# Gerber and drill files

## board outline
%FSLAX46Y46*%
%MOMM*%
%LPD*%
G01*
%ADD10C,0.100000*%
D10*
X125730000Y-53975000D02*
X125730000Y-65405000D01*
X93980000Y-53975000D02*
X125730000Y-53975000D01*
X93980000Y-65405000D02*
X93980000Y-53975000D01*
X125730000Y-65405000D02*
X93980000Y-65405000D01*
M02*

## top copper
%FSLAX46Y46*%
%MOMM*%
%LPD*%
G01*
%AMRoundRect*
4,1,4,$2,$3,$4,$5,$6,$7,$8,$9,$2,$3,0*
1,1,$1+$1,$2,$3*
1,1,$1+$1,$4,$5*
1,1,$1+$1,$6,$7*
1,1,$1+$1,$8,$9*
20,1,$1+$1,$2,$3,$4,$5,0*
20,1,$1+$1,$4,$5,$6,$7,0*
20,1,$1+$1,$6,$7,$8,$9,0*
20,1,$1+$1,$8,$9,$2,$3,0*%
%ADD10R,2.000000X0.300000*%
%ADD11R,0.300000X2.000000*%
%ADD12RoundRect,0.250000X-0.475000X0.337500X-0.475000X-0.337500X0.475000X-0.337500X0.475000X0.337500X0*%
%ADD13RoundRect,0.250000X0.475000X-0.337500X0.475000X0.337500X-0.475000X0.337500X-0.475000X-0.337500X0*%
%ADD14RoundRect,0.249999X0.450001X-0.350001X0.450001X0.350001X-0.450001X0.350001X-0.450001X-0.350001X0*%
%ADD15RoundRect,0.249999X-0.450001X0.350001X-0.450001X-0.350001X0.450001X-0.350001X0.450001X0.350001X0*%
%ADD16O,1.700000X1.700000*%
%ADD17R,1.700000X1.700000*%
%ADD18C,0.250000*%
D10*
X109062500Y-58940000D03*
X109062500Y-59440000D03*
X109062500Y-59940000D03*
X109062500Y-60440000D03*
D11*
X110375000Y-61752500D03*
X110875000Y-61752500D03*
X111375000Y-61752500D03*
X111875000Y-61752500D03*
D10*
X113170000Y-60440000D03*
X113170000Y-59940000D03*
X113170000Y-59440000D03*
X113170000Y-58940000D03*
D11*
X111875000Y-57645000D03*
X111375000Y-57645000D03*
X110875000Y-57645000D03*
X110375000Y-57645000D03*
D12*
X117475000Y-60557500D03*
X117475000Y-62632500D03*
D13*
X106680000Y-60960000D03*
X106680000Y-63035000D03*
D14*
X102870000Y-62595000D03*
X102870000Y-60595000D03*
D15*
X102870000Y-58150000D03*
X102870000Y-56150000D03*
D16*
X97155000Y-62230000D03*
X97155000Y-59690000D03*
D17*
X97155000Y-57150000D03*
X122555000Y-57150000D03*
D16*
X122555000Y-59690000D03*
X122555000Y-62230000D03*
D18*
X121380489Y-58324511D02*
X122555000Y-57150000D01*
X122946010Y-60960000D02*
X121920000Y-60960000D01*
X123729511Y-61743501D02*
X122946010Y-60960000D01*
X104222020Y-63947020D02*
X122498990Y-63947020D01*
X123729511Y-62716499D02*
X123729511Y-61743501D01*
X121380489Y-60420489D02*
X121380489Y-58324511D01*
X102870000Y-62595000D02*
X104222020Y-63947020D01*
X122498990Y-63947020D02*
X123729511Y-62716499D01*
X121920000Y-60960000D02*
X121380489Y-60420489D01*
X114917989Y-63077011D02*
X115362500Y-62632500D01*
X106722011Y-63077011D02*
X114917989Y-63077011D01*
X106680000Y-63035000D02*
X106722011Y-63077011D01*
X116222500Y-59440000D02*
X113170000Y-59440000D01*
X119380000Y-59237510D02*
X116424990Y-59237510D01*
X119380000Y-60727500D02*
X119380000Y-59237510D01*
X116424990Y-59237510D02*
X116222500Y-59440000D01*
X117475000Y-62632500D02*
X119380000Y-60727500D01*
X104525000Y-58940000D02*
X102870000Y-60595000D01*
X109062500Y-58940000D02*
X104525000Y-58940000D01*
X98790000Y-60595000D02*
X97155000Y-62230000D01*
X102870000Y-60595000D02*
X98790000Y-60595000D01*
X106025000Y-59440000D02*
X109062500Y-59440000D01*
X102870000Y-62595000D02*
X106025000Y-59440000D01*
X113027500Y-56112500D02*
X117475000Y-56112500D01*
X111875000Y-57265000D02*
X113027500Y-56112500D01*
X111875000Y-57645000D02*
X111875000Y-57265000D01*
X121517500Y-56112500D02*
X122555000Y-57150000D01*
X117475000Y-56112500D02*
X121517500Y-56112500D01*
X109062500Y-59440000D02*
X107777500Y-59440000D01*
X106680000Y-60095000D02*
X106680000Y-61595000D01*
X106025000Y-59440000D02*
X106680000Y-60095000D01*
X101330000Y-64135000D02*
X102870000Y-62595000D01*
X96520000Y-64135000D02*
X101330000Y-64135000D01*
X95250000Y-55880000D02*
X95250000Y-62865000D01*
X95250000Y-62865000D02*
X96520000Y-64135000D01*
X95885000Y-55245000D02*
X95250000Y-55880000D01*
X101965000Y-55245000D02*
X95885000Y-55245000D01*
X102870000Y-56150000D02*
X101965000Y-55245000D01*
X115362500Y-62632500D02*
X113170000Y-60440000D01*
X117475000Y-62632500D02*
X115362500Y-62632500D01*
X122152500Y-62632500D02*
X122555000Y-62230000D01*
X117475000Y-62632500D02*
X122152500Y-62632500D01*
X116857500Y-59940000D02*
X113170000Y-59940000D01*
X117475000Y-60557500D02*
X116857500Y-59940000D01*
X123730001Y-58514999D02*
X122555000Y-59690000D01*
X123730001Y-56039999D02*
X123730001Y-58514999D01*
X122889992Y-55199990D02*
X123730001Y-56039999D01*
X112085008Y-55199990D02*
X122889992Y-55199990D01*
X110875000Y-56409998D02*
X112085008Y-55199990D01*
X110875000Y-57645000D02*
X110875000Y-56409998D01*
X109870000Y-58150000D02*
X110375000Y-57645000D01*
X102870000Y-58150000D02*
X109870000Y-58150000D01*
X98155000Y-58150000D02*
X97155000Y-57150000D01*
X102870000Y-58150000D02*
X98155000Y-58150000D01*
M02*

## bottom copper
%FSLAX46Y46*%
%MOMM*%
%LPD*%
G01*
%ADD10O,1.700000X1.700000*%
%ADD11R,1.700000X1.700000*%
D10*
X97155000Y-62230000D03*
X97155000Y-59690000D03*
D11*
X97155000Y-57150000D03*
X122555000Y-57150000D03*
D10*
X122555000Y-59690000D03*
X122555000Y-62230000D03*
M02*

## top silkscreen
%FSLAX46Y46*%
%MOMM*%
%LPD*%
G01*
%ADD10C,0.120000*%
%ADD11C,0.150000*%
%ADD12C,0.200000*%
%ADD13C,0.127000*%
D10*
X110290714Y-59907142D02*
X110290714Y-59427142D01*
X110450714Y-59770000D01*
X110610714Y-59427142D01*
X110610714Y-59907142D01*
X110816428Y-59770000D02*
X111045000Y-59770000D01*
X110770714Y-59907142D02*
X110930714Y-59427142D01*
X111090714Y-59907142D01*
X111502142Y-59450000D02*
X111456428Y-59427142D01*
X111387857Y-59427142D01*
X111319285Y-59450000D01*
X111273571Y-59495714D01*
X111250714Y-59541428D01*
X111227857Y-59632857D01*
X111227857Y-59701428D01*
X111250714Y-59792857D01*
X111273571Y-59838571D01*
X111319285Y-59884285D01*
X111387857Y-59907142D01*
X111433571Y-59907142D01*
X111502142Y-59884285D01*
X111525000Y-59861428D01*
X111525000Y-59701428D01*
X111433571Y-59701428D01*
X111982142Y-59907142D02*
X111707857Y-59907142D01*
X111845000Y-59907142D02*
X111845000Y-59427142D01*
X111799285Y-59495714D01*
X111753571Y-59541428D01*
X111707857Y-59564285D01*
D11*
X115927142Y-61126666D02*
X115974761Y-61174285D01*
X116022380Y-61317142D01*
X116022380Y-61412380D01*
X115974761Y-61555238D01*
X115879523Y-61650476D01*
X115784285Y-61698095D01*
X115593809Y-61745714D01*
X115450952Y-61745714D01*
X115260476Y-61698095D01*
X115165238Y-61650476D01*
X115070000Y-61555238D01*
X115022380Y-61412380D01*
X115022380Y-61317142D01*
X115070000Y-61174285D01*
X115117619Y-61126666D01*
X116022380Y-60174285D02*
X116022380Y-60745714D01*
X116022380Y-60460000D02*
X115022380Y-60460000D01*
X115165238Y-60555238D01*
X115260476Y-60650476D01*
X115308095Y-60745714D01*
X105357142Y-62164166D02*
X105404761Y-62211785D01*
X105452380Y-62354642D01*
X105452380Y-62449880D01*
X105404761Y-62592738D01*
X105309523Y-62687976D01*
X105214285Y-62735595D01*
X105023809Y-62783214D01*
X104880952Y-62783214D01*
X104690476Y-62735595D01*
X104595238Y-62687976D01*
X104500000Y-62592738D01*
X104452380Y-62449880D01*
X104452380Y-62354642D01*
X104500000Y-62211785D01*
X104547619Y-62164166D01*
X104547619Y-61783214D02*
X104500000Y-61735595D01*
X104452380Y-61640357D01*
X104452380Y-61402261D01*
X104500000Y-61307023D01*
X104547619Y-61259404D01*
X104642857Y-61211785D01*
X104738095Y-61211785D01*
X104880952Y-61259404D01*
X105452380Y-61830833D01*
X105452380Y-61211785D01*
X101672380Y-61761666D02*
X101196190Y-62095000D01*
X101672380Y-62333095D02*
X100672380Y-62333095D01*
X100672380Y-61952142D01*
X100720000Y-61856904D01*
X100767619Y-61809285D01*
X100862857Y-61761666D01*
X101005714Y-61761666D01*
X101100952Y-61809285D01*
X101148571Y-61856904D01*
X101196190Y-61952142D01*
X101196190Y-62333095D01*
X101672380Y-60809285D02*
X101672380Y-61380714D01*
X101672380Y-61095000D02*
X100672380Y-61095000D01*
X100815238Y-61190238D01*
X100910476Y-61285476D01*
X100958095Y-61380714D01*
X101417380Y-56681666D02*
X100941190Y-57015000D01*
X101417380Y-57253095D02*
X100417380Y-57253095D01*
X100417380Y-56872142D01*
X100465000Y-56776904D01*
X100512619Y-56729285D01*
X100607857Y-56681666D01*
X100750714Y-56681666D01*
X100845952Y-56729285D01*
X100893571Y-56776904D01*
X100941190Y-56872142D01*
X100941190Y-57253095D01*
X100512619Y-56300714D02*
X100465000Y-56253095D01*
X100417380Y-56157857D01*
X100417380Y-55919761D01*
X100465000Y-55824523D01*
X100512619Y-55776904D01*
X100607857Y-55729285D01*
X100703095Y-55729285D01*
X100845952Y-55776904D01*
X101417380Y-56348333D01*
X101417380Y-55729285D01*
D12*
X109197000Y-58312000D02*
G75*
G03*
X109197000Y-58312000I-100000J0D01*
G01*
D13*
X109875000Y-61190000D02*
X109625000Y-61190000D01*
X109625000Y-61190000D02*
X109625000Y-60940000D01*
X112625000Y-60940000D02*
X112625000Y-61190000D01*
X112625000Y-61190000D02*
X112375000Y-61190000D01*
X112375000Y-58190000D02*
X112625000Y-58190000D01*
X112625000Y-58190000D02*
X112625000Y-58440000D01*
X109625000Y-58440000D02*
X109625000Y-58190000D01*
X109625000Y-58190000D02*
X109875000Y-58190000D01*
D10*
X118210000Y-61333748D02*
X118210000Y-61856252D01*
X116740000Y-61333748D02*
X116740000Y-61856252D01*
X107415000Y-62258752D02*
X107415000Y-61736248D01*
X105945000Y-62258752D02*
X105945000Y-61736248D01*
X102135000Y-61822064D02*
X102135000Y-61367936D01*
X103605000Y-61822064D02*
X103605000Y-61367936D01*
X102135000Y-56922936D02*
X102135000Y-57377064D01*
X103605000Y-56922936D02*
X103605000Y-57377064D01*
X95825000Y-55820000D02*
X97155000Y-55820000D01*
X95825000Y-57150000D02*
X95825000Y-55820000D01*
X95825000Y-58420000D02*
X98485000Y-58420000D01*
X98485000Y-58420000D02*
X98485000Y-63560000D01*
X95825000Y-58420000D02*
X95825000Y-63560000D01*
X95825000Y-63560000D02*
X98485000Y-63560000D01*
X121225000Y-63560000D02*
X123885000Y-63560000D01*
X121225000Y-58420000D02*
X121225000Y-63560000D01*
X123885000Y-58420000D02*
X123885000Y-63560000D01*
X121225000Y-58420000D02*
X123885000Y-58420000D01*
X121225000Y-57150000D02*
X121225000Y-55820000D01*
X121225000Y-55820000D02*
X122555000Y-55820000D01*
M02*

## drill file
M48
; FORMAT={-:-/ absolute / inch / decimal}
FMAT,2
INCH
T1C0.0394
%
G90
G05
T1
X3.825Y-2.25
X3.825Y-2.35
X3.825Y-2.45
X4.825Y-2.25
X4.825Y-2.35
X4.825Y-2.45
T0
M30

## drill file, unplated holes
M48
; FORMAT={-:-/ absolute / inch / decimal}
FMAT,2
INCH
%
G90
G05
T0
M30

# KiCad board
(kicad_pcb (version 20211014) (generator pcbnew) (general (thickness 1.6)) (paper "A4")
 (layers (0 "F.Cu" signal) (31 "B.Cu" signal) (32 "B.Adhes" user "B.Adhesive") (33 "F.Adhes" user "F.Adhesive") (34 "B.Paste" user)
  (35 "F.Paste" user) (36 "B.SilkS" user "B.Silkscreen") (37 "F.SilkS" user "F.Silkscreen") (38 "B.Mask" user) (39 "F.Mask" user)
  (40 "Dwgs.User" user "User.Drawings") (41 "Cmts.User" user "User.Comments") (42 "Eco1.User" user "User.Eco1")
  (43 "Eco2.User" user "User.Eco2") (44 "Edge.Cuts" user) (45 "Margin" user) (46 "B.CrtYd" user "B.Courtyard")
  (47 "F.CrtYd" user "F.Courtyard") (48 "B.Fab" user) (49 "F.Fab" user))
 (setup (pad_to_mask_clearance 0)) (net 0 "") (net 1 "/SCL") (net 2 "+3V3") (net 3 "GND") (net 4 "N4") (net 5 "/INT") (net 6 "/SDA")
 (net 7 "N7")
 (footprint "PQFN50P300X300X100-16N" (layer "F.Cu") (at 111.125 59.69)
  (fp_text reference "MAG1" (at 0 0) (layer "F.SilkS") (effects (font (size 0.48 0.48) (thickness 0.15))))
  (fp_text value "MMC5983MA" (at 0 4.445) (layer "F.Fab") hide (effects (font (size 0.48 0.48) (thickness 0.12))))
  (fp_line (start 1.5 1.5) (end 1.25 1.5) (layer "F.SilkS") (width 0.127))
  (fp_line (start 1.5 -1.5) (end 1.5 -1.25) (layer "F.SilkS") (width 0.127))
  (fp_line (start 1.25 -1.5) (end 1.5 -1.5) (layer "F.SilkS") (width 0.127))
  (fp_line (start -1.5 -1.5) (end -1.25 -1.5) (layer "F.SilkS") (width 0.127))
  (fp_line (start -1.5 -1.25) (end -1.5 -1.5) (layer "F.SilkS") (width 0.127))
  (fp_line (start 1.5 1.25) (end 1.5 1.5) (layer "F.SilkS") (width 0.127))
  (fp_line (start -1.25 1.5) (end -1.5 1.5) (layer "F.SilkS") (width 0.127))
  (fp_line (start -1.5 1.5) (end -1.5 1.25) (layer "F.SilkS") (width 0.127))
  (fp_circle (center -2.028 -1.378) (end -1.928 -1.378) (layer "F.SilkS") (width 0.2) (fill none))
  (pad "1" smd rect locked (at -2.0625 -0.75) (size 2 0.3) (layers "F.Cu" "F.Paste" "F.Mask") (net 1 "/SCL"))
  (pad "2" smd rect locked (at -2.0625 -0.25) (size 2 0.3) (layers "F.Cu" "F.Paste" "F.Mask") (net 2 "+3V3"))
  (pad "3" smd rect locked (at -2.0625 0.25) (size 2 0.3) (layers "F.Cu" "F.Paste" "F.Mask"))
  (pad "4" smd rect locked (at -2.0625 0.75) (size 2 0.3) (layers "F.Cu" "F.Paste" "F.Mask"))
  (pad "5" smd rect locked (at -0.75 2.0625) (size 0.3 2) (layers "F.Cu" "F.Paste" "F.Mask"))
  (pad "6" smd rect locked (at -0.25 2.0625) (size 0.3 2) (layers "F.Cu" "F.Paste" "F.Mask"))
  (pad "7" smd rect locked (at 0.25 2.0625) (size 0.3 2) (layers "F.Cu" "F.Paste" "F.Mask"))
  (pad "8" smd rect locked (at 0.75 2.0625) (size 0.3 2) (layers "F.Cu" "F.Paste" "F.Mask"))
  (pad "9" smd rect locked (at 2.045 0.75) (size 2 0.3) (layers "F.Cu" "F.Paste" "F.Mask") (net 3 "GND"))
  (pad "10" smd rect locked (at 2.045 0.25) (size 2 0.3) (layers "F.Cu" "F.Paste" "F.Mask") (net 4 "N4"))
  (pad "11" smd rect locked (at 2.045 -0.25) (size 2 0.3) (layers "F.Cu" "F.Paste" "F.Mask") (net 3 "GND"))
  (pad "12" smd rect locked (at 2.045 -0.75) (size 2 0.3) (layers "F.Cu" "F.Paste" "F.Mask"))
  (pad "13" smd rect locked (at 0.75 -2.045) (size 0.3 2) (layers "F.Cu" "F.Paste" "F.Mask") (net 2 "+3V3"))
  (pad "14" smd rect locked (at 0.25 -2.045) (size 0.3 2) (layers "F.Cu" "F.Paste" "F.Mask"))
  (pad "15" smd rect locked (at -0.25 -2.045) (size 0.3 2) (layers "F.Cu" "F.Paste" "F.Mask") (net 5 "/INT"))
  (pad "16" smd rect locked (at -0.75 -2.045) (size 0.3 2) (layers "F.Cu" "F.Paste" "F.Mask") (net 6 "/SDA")))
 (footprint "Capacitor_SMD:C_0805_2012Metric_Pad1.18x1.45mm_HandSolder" (layer "F.Cu") (at 117.475 61.595 -90)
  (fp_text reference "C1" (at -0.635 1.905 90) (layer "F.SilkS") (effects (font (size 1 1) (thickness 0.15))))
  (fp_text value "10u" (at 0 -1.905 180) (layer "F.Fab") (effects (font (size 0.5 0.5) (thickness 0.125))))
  (fp_line (start -0.261252 -0.735) (end 0.261252 -0.735) (layer "F.SilkS") (width 0.12))
  (fp_line (start -0.261252 0.735) (end 0.261252 0.735) (layer "F.SilkS") (width 0.12))
  (pad "1" smd roundrect locked (at -1.0375 0 270) (size 1.175 1.45) (layers "F.Cu" "F.Paste" "F.Mask") (roundrect_rratio 0.2127659574)
   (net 4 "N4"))
  (pad "2" smd roundrect locked (at 1.0375 0 270) (size 1.175 1.45) (layers "F.Cu" "F.Paste" "F.Mask") (roundrect_rratio 0.2127659574)
   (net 3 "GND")))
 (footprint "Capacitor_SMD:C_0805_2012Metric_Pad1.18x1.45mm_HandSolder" (layer "F.Cu") (at 106.68 61.9975 90)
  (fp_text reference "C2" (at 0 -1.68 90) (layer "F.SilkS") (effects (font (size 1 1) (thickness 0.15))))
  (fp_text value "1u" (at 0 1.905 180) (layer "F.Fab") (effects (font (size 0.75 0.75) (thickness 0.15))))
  (fp_line (start -0.261252 -0.735) (end 0.261252 -0.735) (layer "F.SilkS") (width 0.12))
  (fp_line (start -0.261252 0.735) (end 0.261252 0.735) (layer "F.SilkS") (width 0.12))
  (pad "1" smd roundrect locked (at -1.0375 0 90) (size 1.175 1.45) (layers "F.Cu" "F.Paste" "F.Mask") (roundrect_rratio 0.2127659574)
   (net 3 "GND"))
  (pad "2" smd roundrect locked (at 1.0375 0 90) (size 1.175 1.45) (layers "F.Cu" "F.Paste" "F.Mask") (roundrect_rratio 0.2127659574)
   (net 2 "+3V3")))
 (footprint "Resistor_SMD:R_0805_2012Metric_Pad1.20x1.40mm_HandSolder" (layer "F.Cu") (at 102.87 61.595 90)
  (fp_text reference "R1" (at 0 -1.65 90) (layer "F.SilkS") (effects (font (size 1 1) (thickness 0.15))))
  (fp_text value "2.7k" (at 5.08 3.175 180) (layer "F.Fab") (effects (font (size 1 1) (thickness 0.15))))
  (fp_line (start -0.227064 -0.735) (end 0.227064 -0.735) (layer "F.SilkS") (width 0.12))
  (fp_line (start -0.227064 0.735) (end 0.227064 0.735) (layer "F.SilkS") (width 0.12))
  (pad "1" smd roundrect locked (at -1 0 90) (size 1.2 1.4) (layers "F.Cu" "F.Paste" "F.Mask") (roundrect_rratio 0.2083325) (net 2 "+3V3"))
  (pad "2" smd roundrect locked (at 1 0 90) (size 1.2 1.4) (layers "F.Cu" "F.Paste" "F.Mask") (roundrect_rratio 0.2083325) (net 1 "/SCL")))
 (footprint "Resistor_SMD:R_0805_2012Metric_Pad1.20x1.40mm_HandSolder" (layer "F.Cu") (at 102.87 57.15 -90)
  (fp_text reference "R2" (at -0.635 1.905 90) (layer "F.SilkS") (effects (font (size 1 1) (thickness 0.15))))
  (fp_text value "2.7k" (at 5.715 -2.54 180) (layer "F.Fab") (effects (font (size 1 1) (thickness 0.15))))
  (fp_line (start -0.227064 -0.735) (end 0.227064 -0.735) (layer "F.SilkS") (width 0.12))
  (fp_line (start -0.227064 0.735) (end 0.227064 0.735) (layer "F.SilkS") (width 0.12))
  (pad "1" smd roundrect locked (at -1 0 270) (size 1.2 1.4) (layers "F.Cu" "F.Paste" "F.Mask") (roundrect_rratio 0.2083325) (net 2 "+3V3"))
  (pad "2" smd roundrect locked (at 1 0 270) (size 1.2 1.4) (layers "F.Cu" "F.Paste" "F.Mask") (roundrect_rratio 0.2083325) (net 6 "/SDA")))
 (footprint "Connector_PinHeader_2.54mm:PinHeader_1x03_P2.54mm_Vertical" (layer "F.Cu") (at 97.155 57.15)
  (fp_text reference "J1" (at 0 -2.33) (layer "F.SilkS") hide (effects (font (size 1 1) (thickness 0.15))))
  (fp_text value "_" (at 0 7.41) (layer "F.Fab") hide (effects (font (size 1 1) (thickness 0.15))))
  (fp_line (start -1.33 1.27) (end -1.33 6.41) (layer "F.SilkS") (width 0.12))
  (fp_line (start -1.33 1.27) (end 1.33 1.27) (layer "F.SilkS") (width 0.12))
  (fp_line (start -1.33 -1.33) (end 0 -1.33) (layer "F.SilkS") (width 0.12))
  (fp_line (start -1.33 0) (end -1.33 -1.33) (layer "F.SilkS") (width 0.12))
  (fp_line (start 1.33 1.27) (end 1.33 6.41) (layer "F.SilkS") (width 0.12))
  (fp_line (start -1.33 6.41) (end 1.33 6.41) (layer "F.SilkS") (width 0.12))
  (pad "1" thru_hole rect locked (at 0 0) (size 1.7 1.7) (drill 1) (layers *.Cu *.Mask) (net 6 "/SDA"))
  (pad "2" thru_hole oval locked (at 0 2.54) (size 1.7 1.7) (drill 1) (layers *.Cu *.Mask) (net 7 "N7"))
  (pad "3" thru_hole oval locked (at 0 5.08) (size 1.7 1.7) (drill 1) (layers *.Cu *.Mask) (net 1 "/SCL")))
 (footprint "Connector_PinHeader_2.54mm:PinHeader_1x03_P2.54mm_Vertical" (layer "F.Cu") (at 122.555 57.15)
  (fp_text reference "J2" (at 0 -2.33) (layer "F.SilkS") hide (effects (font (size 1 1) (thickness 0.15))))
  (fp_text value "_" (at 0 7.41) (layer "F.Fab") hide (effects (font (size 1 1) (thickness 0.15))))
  (fp_line (start -1.33 6.41) (end 1.33 6.41) (layer "F.SilkS") (width 0.12))
  (fp_line (start -1.33 1.27) (end -1.33 6.41) (layer "F.SilkS") (width 0.12))
  (fp_line (start -1.33 -1.33) (end 0 -1.33) (layer "F.SilkS") (width 0.12))
  (fp_line (start -1.33 0) (end -1.33 -1.33) (layer "F.SilkS") (width 0.12))
  (fp_line (start -1.33 1.27) (end 1.33 1.27) (layer "F.SilkS") (width 0.12))
  (fp_line (start 1.33 1.27) (end 1.33 6.41) (layer "F.SilkS") (width 0.12))
  (pad "1" thru_hole rect locked (at 0 0) (size 1.7 1.7) (drill 1) (layers *.Cu *.Mask) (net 2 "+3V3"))
  (pad "2" thru_hole oval locked (at 0 2.54) (size 1.7 1.7) (drill 1) (layers *.Cu *.Mask) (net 5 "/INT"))
  (pad "3" thru_hole oval locked (at 0 5.08) (size 1.7 1.7) (drill 1) (layers *.Cu *.Mask) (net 3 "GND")))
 (gr_line (start 93.98 53.975) (end 125.73 53.975) (layer "Edge.Cuts") (width 0.1))
 (gr_line (start 125.73 53.975) (end 125.73 65.405) (layer "Edge.Cuts") (width 0.1))
 (gr_line (start 125.73 65.405) (end 93.98 65.405) (layer "Edge.Cuts") (width 0.1))
 (gr_line (start 93.98 65.405) (end 93.98 53.975) (layer "Edge.Cuts") (width 0.1))
 (segment (start 104.525 58.94) (end 102.87 60.595) (width 0.25) (layer "F.Cu") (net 1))
 (segment (start 102.87 60.595) (end 98.79 60.595) (width 0.25) (layer "F.Cu") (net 1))
 (segment (start 98.79 60.595) (end 97.155 62.23) (width 0.25) (layer "F.Cu") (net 1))
 (segment (start 109.0625 58.94) (end 104.525 58.94) (width 0.25) (layer "F.Cu") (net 1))
 (segment (start 101.965 55.245) (end 95.885 55.245) (width 0.25) (layer "F.Cu") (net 2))
 (segment (start 111.875 57.265) (end 113.0275 56.1125) (width 0.25) (layer "F.Cu") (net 2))
 (segment (start 121.380489 60.420489) (end 121.380489 58.324511) (width 0.25) (layer "F.Cu") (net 2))
 (segment (start 117.475 56.1125) (end 121.5175 56.1125) (width 0.25) (layer "F.Cu") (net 2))
 (segment (start 96.52 64.135) (end 101.33 64.135) (width 0.25) (layer "F.Cu") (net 2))
 (segment (start 109.0625 59.44) (end 107.7775 59.44) (width 0.25) (layer "F.Cu") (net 2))
 (segment (start 104.22202 63.94702) (end 122.49899 63.94702) (width 0.25) (layer "F.Cu") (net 2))
 (segment (start 111.875 57.645) (end 111.875 57.265) (width 0.25) (layer "F.Cu") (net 2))
 (segment (start 102.87 56.15) (end 101.965 55.245) (width 0.25) (layer "F.Cu") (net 2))
 (segment (start 123.729511 62.716499) (end 123.729511 61.743501) (width 0.25) (layer "F.Cu") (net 2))
 (segment (start 122.49899 63.94702) (end 123.729511 62.716499) (width 0.25) (layer "F.Cu") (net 2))
 (segment (start 95.25 62.865) (end 96.52 64.135) (width 0.25) (layer "F.Cu") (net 2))
 (segment (start 101.33 64.135) (end 102.87 62.595) (width 0.25) (layer "F.Cu") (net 2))
 (segment (start 102.87 62.595) (end 104.22202 63.94702) (width 0.25) (layer "F.Cu") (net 2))
 (segment (start 113.0275 56.1125) (end 117.475 56.1125) (width 0.25) (layer "F.Cu") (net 2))
 (segment (start 95.25 55.88) (end 95.25 62.865) (width 0.25) (layer "F.Cu") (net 2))
 (segment (start 106.025 59.44) (end 109.0625 59.44) (width 0.25) (layer "F.Cu") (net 2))
 (segment (start 95.885 55.245) (end 95.25 55.88) (width 0.25) (layer "F.Cu") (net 2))
 (segment (start 106.025 59.44) (end 106.68 60.095) (width 0.25) (layer "F.Cu") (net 2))
 (segment (start 102.87 62.595) (end 106.025 59.44) (width 0.25) (layer "F.Cu") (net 2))
 (segment (start 121.92 60.96) (end 121.380489 60.420489) (width 0.25) (layer "F.Cu") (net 2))
 (segment (start 106.68 60.095) (end 106.68 61.595) (width 0.25) (layer "F.Cu") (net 2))
 (segment (start 121.380489 58.324511) (end 122.555 57.15) (width 0.25) (layer "F.Cu") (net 2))
 (segment (start 121.5175 56.1125) (end 122.555 57.15) (width 0.25) (layer "F.Cu") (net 2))
 (segment (start 122.94601 60.96) (end 121.92 60.96) (width 0.25) (layer "F.Cu") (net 2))
 (segment (start 123.729511 61.743501) (end 122.94601 60.96) (width 0.25) (layer "F.Cu") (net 2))
 (segment (start 119.38 60.7275) (end 119.38 59.23751) (width 0.25) (layer "F.Cu") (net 3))
 (segment (start 106.722011 63.077011) (end 114.917989 63.077011) (width 0.25) (layer "F.Cu") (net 3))
 (segment (start 106.68 63.035) (end 106.722011 63.077011) (width 0.25) (layer "F.Cu") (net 3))
 (segment (start 119.38 59.23751) (end 116.42499 59.23751) (width 0.25) (layer "F.Cu") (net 3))
 (segment (start 117.475 62.6325) (end 122.1525 62.6325) (width 0.25) (layer "F.Cu") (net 3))
 (segment (start 117.475 62.6325) (end 119.38 60.7275) (width 0.25) (layer "F.Cu") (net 3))
 (segment (start 115.3625 62.6325) (end 113.17 60.44) (width 0.25) (layer "F.Cu") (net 3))
 (segment (start 116.2225 59.44) (end 113.17 59.44) (width 0.25) (layer "F.Cu") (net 3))
 (segment (start 122.1525 62.6325) (end 122.555 62.23) (width 0.25) (layer "F.Cu") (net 3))
 (segment (start 114.917989 63.077011) (end 115.3625 62.6325) (width 0.25) (layer "F.Cu") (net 3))
 (segment (start 116.42499 59.23751) (end 116.2225 59.44) (width 0.25) (layer "F.Cu") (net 3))
 (segment (start 117.475 62.6325) (end 115.3625 62.6325) (width 0.25) (layer "F.Cu") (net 3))
 (segment (start 117.475 60.5575) (end 116.8575 59.94) (width 0.25) (layer "F.Cu") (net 4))
 (segment (start 116.8575 59.94) (end 113.17 59.94) (width 0.25) (layer "F.Cu") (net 4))
 (segment (start 112.085008 55.19999) (end 122.889992 55.19999) (width 0.25) (layer "F.Cu") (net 5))
 (segment (start 123.730001 58.514999) (end 122.555 59.69) (width 0.25) (layer "F.Cu") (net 5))
 (segment (start 110.875 57.645) (end 110.875 56.409998) (width 0.25) (layer "F.Cu") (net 5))
 (segment (start 123.730001 56.039999) (end 123.730001 58.514999) (width 0.25) (layer "F.Cu") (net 5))
 (segment (start 122.889992 55.19999) (end 123.730001 56.039999) (width 0.25) (layer "F.Cu") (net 5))
 (segment (start 110.875 56.409998) (end 112.085008 55.19999) (width 0.25) (layer "F.Cu") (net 5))
 (segment (start 109.87 58.15) (end 110.375 57.645) (width 0.25) (layer "F.Cu") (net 6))
 (segment (start 98.155 58.15) (end 97.155 57.15) (width 0.25) (layer "F.Cu") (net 6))
 (segment (start 102.87 58.15) (end 109.87 58.15) (width 0.25) (layer "F.Cu") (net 6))
 (segment (start 102.87 58.15) (end 98.155 58.15) (width 0.25) (layer "F.Cu") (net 6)))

